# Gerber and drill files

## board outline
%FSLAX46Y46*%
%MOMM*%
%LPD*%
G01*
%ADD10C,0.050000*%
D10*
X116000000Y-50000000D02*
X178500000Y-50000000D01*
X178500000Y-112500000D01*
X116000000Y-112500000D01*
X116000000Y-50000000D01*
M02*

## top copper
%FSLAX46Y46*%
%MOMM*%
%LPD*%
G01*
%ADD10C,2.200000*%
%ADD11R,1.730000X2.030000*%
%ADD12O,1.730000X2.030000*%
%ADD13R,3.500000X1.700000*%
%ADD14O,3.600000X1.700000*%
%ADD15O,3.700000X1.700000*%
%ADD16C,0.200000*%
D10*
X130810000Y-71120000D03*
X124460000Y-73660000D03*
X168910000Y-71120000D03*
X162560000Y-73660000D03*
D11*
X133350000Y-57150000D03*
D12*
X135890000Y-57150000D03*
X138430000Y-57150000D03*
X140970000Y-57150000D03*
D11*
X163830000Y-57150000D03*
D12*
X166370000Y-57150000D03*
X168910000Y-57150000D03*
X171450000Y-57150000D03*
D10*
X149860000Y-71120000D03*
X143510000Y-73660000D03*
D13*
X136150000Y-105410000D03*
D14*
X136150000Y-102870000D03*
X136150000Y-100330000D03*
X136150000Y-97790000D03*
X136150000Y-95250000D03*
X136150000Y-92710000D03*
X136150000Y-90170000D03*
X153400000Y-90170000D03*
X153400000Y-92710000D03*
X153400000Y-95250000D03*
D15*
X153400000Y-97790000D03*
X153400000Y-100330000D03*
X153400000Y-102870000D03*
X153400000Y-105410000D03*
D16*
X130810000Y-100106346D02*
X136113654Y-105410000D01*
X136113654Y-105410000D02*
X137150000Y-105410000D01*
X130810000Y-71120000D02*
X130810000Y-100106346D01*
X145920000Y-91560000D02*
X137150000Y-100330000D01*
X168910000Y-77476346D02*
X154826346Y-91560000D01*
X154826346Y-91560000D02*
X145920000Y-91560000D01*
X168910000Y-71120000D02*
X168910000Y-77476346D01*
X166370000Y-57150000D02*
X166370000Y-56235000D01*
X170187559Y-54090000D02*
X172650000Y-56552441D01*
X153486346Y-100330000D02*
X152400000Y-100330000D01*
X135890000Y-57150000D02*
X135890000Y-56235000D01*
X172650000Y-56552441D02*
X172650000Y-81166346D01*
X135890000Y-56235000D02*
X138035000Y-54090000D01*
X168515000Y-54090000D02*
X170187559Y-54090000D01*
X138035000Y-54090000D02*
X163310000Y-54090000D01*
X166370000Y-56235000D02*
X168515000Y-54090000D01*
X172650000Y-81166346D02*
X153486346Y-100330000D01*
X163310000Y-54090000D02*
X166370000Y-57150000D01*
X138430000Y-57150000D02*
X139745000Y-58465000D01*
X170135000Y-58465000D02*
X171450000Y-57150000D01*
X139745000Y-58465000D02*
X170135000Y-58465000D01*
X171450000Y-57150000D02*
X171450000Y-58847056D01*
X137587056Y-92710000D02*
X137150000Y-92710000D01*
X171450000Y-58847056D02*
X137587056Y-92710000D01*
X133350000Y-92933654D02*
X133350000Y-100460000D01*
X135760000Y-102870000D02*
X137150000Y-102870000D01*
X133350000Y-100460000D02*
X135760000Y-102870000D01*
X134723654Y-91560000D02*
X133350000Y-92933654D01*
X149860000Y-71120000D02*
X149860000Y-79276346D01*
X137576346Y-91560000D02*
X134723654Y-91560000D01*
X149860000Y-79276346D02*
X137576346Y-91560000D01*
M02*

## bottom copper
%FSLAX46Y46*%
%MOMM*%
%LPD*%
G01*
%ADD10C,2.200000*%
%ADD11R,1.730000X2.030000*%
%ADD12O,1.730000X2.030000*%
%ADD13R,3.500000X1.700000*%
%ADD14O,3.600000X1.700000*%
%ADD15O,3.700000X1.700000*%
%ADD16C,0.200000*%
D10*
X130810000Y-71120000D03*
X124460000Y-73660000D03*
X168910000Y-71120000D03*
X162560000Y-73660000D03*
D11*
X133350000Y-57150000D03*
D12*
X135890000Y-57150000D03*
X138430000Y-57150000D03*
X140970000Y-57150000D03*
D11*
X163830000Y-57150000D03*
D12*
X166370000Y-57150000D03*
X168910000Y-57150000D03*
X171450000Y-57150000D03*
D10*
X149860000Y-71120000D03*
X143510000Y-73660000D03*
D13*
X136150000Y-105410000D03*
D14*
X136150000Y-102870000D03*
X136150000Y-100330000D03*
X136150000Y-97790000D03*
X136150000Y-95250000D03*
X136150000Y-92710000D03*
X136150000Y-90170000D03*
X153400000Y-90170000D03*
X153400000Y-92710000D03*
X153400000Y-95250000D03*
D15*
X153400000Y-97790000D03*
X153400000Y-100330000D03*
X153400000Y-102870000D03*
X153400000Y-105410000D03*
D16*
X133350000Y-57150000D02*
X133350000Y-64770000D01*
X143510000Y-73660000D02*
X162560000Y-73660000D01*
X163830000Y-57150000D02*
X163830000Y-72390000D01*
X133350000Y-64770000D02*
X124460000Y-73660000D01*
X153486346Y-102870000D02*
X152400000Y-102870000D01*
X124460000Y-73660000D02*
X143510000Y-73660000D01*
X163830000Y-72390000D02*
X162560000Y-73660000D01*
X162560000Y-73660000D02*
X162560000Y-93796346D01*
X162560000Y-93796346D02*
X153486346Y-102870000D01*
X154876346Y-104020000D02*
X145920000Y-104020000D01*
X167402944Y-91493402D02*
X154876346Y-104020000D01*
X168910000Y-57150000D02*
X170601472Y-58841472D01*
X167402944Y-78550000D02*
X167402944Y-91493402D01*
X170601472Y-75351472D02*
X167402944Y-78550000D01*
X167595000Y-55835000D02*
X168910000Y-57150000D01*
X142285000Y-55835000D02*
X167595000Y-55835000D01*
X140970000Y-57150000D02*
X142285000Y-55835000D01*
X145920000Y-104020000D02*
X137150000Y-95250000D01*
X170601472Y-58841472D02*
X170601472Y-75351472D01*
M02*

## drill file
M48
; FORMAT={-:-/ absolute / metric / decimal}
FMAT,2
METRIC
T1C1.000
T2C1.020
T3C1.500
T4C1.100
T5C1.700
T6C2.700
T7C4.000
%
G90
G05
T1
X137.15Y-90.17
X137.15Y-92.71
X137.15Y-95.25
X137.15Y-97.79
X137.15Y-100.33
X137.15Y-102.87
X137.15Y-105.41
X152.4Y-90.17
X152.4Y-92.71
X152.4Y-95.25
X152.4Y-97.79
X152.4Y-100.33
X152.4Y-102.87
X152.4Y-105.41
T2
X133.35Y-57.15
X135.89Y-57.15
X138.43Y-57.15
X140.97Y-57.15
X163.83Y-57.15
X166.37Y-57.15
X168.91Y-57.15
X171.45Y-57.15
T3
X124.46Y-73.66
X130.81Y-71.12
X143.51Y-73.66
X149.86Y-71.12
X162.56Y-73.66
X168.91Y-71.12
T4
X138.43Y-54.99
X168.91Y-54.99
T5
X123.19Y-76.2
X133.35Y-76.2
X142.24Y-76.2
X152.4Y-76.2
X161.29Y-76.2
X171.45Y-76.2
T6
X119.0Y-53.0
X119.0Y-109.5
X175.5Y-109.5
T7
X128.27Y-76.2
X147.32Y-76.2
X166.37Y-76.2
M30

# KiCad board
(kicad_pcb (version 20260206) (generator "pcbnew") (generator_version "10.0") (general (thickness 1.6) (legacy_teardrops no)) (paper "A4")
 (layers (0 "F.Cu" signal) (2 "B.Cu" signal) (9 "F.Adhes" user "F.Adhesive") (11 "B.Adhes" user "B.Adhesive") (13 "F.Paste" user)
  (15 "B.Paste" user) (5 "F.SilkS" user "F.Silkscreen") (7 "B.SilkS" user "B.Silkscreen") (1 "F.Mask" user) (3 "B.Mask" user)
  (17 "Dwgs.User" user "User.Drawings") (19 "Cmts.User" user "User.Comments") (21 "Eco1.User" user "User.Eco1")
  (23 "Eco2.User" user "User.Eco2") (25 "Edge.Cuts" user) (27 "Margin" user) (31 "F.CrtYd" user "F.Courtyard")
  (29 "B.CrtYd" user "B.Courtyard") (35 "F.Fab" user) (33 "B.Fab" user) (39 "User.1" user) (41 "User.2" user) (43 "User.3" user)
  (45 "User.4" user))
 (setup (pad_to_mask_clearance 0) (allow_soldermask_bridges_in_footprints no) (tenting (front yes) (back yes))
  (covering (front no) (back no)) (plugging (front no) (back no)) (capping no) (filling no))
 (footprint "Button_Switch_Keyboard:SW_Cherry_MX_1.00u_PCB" (layer "F.Cu") (at 130.81 71.12)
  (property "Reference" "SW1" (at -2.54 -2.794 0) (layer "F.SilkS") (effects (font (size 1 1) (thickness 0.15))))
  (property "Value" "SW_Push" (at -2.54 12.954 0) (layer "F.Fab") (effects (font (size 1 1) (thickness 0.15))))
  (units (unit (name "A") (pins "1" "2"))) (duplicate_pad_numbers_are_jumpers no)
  (pad "" np_thru_hole circle (at -7.62 5.08) (size 1.7 1.7) (drill 1.7) (layers "*.Cu" "*.Mask"))
  (pad "" np_thru_hole circle (at -2.54 5.08) (size 4 4) (drill 4) (layers "*.Cu" "*.Mask"))
  (pad "" np_thru_hole circle (at 2.54 5.08) (size 1.7 1.7) (drill 1.7) (layers "*.Cu" "*.Mask"))
  (pad "1" thru_hole circle (at 0 0) (size 2.2 2.2) (drill 1.5) (layers "*.Cu" "*.Mask") (remove_unused_layers no) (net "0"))
  (pad "2" thru_hole circle (at -6.35 2.54) (size 2.2 2.2) (drill 1.5) (layers "*.Cu" "*.Mask") (remove_unused_layers no) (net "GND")))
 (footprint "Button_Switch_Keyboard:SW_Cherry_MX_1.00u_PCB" (layer "F.Cu") (at 168.91 71.12)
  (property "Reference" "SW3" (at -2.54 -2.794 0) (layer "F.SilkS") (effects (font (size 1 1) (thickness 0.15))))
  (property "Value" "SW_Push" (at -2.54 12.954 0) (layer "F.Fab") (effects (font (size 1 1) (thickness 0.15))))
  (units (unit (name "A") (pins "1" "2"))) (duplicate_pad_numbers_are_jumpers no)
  (pad "" np_thru_hole circle (at -7.62 5.08) (size 1.7 1.7) (drill 1.7) (layers "*.Cu" "*.Mask"))
  (pad "" np_thru_hole circle (at -2.54 5.08) (size 4 4) (drill 4) (layers "*.Cu" "*.Mask"))
  (pad "" np_thru_hole circle (at 2.54 5.08) (size 1.7 1.7) (drill 1.7) (layers "*.Cu" "*.Mask"))
  (pad "1" thru_hole circle (at 0 0) (size 2.2 2.2) (drill 1.5) (layers "*.Cu" "*.Mask") (remove_unused_layers no) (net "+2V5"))
  (pad "2" thru_hole circle (at -6.35 2.54) (size 2.2 2.2) (drill 1.5) (layers "*.Cu" "*.Mask") (remove_unused_layers no) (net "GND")))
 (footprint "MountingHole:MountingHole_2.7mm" (layer "F.Cu") (at 119 109.5)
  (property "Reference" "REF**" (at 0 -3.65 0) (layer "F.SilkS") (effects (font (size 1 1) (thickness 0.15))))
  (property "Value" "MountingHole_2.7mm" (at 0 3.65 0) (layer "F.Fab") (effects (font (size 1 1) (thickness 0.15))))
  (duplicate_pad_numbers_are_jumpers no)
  (pad "" np_thru_hole circle (at 0 0) (size 2.7 2.7) (drill 2.7) (layers "*.Cu" "*.Mask")))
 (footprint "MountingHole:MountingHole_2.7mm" (layer "F.Cu") (at 175.5 109.5)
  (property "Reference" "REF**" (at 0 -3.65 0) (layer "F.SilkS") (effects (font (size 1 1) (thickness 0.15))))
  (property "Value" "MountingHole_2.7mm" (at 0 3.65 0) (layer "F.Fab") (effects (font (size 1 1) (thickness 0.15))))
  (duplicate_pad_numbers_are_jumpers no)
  (pad "" np_thru_hole circle (at 0 0) (size 2.7 2.7) (drill 2.7) (layers "*.Cu" "*.Mask")))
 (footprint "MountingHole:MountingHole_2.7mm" (layer "F.Cu") (at 119 53)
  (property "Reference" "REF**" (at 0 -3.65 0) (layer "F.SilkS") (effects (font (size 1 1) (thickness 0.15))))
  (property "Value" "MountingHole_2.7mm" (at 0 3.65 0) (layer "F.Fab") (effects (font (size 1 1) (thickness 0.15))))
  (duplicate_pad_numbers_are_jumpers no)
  (pad "" np_thru_hole circle (at 0 0) (size 2.7 2.7) (drill 2.7) (layers "*.Cu" "*.Mask")))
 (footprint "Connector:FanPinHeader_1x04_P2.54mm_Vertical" (layer "F.Cu") (at 133.35 57.15)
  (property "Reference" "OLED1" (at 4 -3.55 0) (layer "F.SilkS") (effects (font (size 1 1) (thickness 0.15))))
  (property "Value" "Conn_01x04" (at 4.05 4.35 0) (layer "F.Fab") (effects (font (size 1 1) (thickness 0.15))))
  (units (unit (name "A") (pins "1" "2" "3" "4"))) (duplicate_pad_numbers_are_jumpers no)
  (pad "" np_thru_hole circle (at 5.08 -2.16 90) (size 1.1 1.1) (drill 1.1) (layers "*.Cu" "*.Mask"))
  (pad "1" thru_hole rect (at 0 0 90) (size 2.03 1.73) (drill 1.02) (layers "*.Cu" "*.Mask") (remove_unused_layers no) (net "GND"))
  (pad "2" thru_hole oval (at 2.54 0 90) (size 2.03 1.73) (drill 1.02) (layers "*.Cu" "*.Mask") (remove_unused_layers no) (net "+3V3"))
  (pad "3" thru_hole oval (at 5.08 0 90) (size 2.03 1.73) (drill 1.02) (layers "*.Cu" "*.Mask") (remove_unused_layers no) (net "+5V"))
  (pad "4" thru_hole oval (at 7.62 0 90) (size 2.03 1.73) (drill 1.02) (layers "*.Cu" "*.Mask") (remove_unused_layers no) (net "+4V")))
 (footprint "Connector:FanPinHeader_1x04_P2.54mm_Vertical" (layer "F.Cu") (at 163.83 57.15)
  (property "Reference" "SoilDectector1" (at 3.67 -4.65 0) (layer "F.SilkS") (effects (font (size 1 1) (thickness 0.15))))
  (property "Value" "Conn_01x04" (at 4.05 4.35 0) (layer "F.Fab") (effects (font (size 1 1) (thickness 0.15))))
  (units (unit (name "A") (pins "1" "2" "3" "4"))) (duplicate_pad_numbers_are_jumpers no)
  (pad "" np_thru_hole circle (at 5.08 -2.16 90) (size 1.1 1.1) (drill 1.1) (layers "*.Cu" "*.Mask"))
  (pad "1" thru_hole rect (at 0 0 90) (size 2.03 1.73) (drill 1.02) (layers "*.Cu" "*.Mask") (remove_unused_layers no) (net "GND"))
  (pad "2" thru_hole oval (at 2.54 0 90) (size 2.03 1.73) (drill 1.02) (layers "*.Cu" "*.Mask") (remove_unused_layers no) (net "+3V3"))
  (pad "3" thru_hole oval (at 5.08 0 90) (size 2.03 1.73) (drill 1.02) (layers "*.Cu" "*.Mask") (remove_unused_layers no) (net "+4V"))
  (pad "4" thru_hole oval (at 7.62 0 90) (size 2.03 1.73) (drill 1.02) (layers "*.Cu" "*.Mask") (remove_unused_layers no) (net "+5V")))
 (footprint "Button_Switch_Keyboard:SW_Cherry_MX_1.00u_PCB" (layer "F.Cu") (at 149.86 71.12)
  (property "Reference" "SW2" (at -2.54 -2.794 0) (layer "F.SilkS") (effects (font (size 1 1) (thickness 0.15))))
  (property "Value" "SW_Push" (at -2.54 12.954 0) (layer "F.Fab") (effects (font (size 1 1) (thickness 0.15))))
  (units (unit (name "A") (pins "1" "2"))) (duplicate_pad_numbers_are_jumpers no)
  (pad "" np_thru_hole circle (at -7.62 5.08) (size 1.7 1.7) (drill 1.7) (layers "*.Cu" "*.Mask"))
  (pad "" np_thru_hole circle (at -2.54 5.08) (size 4 4) (drill 4) (layers "*.Cu" "*.Mask"))
  (pad "" np_thru_hole circle (at 2.54 5.08) (size 1.7 1.7) (drill 1.7) (layers "*.Cu" "*.Mask"))
  (pad "1" thru_hole circle (at 0 0) (size 2.2 2.2) (drill 1.5) (layers "*.Cu" "*.Mask") (remove_unused_layers no) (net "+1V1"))
  (pad "2" thru_hole circle (at -6.35 2.54) (size 2.2 2.2) (drill 1.5) (layers "*.Cu" "*.Mask") (remove_unused_layers no) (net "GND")))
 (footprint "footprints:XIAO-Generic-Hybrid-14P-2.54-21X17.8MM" (layer "B.Cu") (at 144.775 97.79)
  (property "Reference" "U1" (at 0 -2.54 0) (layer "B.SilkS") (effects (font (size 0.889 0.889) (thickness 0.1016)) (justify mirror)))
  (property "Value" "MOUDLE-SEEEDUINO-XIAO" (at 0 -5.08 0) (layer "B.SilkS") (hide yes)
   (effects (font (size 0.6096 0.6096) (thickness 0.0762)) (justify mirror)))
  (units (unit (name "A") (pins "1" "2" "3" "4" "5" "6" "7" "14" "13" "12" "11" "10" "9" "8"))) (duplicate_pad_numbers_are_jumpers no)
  (pad "1" thru_hole rect (at -7.625 7.62) (size 3.5 1.7) (drill 1 (offset -1 0)) (layers "*.Cu" "*.Mask") (remove_unused_layers no)
   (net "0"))
  (pad "2" thru_hole oval (at -7.625 5.08) (size 3.6 1.7) (drill 1 (offset -1 0)) (layers "*.Cu" "*.Mask") (remove_unused_layers no)
   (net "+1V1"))
  (pad "3" thru_hole oval (at -7.625 2.54) (size 3.6 1.7) (drill 1 (offset -1 0)) (layers "*.Cu" "*.Mask") (remove_unused_layers no)
   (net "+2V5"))
  (pad "4" thru_hole oval (at -7.625 0) (size 3.6 1.7) (drill 1 (offset -1 0)) (layers "*.Cu" "*.Mask") (remove_unused_layers no)
   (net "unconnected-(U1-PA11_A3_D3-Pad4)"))
  (pad "5" thru_hole oval (at -7.625 -2.54) (size 3.6 1.7) (drill 1 (offset -1 0)) (layers "*.Cu" "*.Mask") (remove_unused_layers no)
   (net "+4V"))
  (pad "6" thru_hole oval (at -7.625 -5.08 180) (size 3.6 1.7) (drill 1 (offset 1 0)) (layers "*.Cu" "*.Mask") (remove_unused_layers no)
   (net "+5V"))
  (pad "7" thru_hole oval (at -7.625 -7.62) (size 3.6 1.7) (drill 1 (offset -1 0)) (layers "*.Cu" "*.Mask") (remove_unused_layers no)
   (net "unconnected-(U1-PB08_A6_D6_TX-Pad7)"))
  (pad "8" thru_hole oval (at 7.625 -7.62) (size 3.6 1.7) (drill 1 (offset 1 0)) (layers "*.Cu" "*.Mask") (remove_unused_layers no)
   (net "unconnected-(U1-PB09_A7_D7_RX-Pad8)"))
  (pad "9" thru_hole oval (at 7.625 -5.08) (size 3.6 1.7) (drill 1 (offset 1 0)) (layers "*.Cu" "*.Mask") (remove_unused_layers no)
   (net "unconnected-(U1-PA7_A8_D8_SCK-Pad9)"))
  (pad "10" thru_hole oval (at 7.625 -2.54) (size 3.6 1.7) (drill 1 (offset 1 0)) (layers "*.Cu" "*.Mask") (remove_unused_layers no)
   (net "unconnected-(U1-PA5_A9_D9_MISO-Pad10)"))
  (pad "11" thru_hole oval (at 7.625 0) (size 3.7 1.7) (drill 1 (offset 1 0)) (layers "*.Cu" "*.Mask") (remove_unused_layers no)
   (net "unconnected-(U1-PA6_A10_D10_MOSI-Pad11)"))
  (pad "12" thru_hole oval (at 7.625 2.54) (size 3.7 1.7) (drill 1 (offset 1 0)) (layers "*.Cu" "*.Mask") (remove_unused_layers no)
   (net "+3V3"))
  (pad "13" thru_hole oval (at 7.625 5.08) (size 3.7 1.7) (drill 1 (offset 1 0)) (layers "*.Cu" "*.Mask") (remove_unused_layers no)
   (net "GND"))
  (pad "14" thru_hole oval (at 7.625 7.62) (size 3.7 1.7) (drill 1 (offset 1 0)) (layers "*.Cu" "*.Mask") (remove_unused_layers no)
   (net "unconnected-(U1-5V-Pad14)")))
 (gr_rect (start 116 50) (end 178.5 112.5) (stroke (width 0.05) (type default)) (fill no) (layer "Edge.Cuts"))
 (segment (start 130.81 100.106346) (end 136.113654 105.41) (width 0.2) (layer "F.Cu") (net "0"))
 (segment (start 136.113654 105.41) (end 137.15 105.41) (width 0.2) (layer "F.Cu") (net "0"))
 (segment (start 130.81 71.12) (end 130.81 100.106346) (width 0.2) (layer "F.Cu") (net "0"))
 (segment (start 133.35 57.15) (end 133.35 64.77) (width 0.2) (layer "B.Cu") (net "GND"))
 (segment (start 143.51 73.66) (end 162.56 73.66) (width 0.2) (layer "B.Cu") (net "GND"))
 (segment (start 163.83 57.15) (end 163.83 72.39) (width 0.2) (layer "B.Cu") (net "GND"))
 (segment (start 133.35 64.77) (end 124.46 73.66) (width 0.2) (layer "B.Cu") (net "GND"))
 (segment (start 153.486346 102.87) (end 152.4 102.87) (width 0.2) (layer "B.Cu") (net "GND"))
 (segment (start 124.46 73.66) (end 143.51 73.66) (width 0.2) (layer "B.Cu") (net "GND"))
 (segment (start 163.83 72.39) (end 162.56 73.66) (width 0.2) (layer "B.Cu") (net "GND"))
 (segment (start 162.56 73.66) (end 162.56 93.796346) (width 0.2) (layer "B.Cu") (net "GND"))
 (segment (start 162.56 93.796346) (end 153.486346 102.87) (width 0.2) (layer "B.Cu") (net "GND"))
 (segment (start 145.92 91.56) (end 137.15 100.33) (width 0.2) (layer "F.Cu") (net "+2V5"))
 (segment (start 168.91 77.476346) (end 154.826346 91.56) (width 0.2) (layer "F.Cu") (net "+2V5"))
 (segment (start 154.826346 91.56) (end 145.92 91.56) (width 0.2) (layer "F.Cu") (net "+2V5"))
 (segment (start 168.91 71.12) (end 168.91 77.476346) (width 0.2) (layer "F.Cu") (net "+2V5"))
 (segment (start 166.37 57.15) (end 166.37 56.235) (width 0.2) (layer "F.Cu") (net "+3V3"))
 (segment (start 170.187559 54.09) (end 172.65 56.552441) (width 0.2) (layer "F.Cu") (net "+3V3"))
 (segment (start 153.486346 100.33) (end 152.4 100.33) (width 0.2) (layer "F.Cu") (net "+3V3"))
 (segment (start 135.89 57.15) (end 135.89 56.235) (width 0.2) (layer "F.Cu") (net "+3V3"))
 (segment (start 172.65 56.552441) (end 172.65 81.166346) (width 0.2) (layer "F.Cu") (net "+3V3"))
 (segment (start 135.89 56.235) (end 138.035 54.09) (width 0.2) (layer "F.Cu") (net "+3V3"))
 (segment (start 168.515 54.09) (end 170.187559 54.09) (width 0.2) (layer "F.Cu") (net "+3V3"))
 (segment (start 138.035 54.09) (end 163.31 54.09) (width 0.2) (layer "F.Cu") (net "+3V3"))
 (segment (start 166.37 56.235) (end 168.515 54.09) (width 0.2) (layer "F.Cu") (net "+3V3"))
 (segment (start 172.65 81.166346) (end 153.486346 100.33) (width 0.2) (layer "F.Cu") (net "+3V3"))
 (segment (start 163.31 54.09) (end 166.37 57.15) (width 0.2) (layer "F.Cu") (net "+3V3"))
 (segment (start 138.43 57.15) (end 139.745 58.465) (width 0.2) (layer "F.Cu") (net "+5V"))
 (segment (start 170.135 58.465) (end 171.45 57.15) (width 0.2) (layer "F.Cu") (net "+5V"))
 (segment (start 139.745 58.465) (end 170.135 58.465) (width 0.2) (layer "F.Cu") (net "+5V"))
 (segment (start 171.45 57.15) (end 171.45 58.847056) (width 0.2) (layer "F.Cu") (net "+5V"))
 (segment (start 137.587056 92.71) (end 137.15 92.71) (width 0.2) (layer "F.Cu") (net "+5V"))
 (segment (start 171.45 58.847056) (end 137.587056 92.71) (width 0.2) (layer "F.Cu") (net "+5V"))
 (segment (start 154.876346 104.02) (end 145.92 104.02) (width 0.2) (layer "B.Cu") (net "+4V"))
 (segment (start 167.402944 91.493402) (end 154.876346 104.02) (width 0.2) (layer "B.Cu") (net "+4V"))
 (segment (start 168.91 57.15) (end 170.601472 58.841472) (width 0.2) (layer "B.Cu") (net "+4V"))
 (segment (start 167.402944 78.55) (end 167.402944 91.493402) (width 0.2) (layer "B.Cu") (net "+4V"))
 (segment (start 170.601472 75.351472) (end 167.402944 78.55) (width 0.2) (layer "B.Cu") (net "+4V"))
 (segment (start 167.595 55.835) (end 168.91 57.15) (width 0.2) (layer "B.Cu") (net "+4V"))
 (segment (start 142.285 55.835) (end 167.595 55.835) (width 0.2) (layer "B.Cu") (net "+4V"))
 (segment (start 140.97 57.15) (end 142.285 55.835) (width 0.2) (layer "B.Cu") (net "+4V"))
 (segment (start 145.92 104.02) (end 137.15 95.25) (width 0.2) (layer "B.Cu") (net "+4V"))
 (segment (start 170.601472 58.841472) (end 170.601472 75.351472) (width 0.2) (layer "B.Cu") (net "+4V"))
 (segment (start 133.35 92.933654) (end 133.35 100.46) (width 0.2) (layer "F.Cu") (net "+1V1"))
 (segment (start 135.76 102.87) (end 137.15 102.87) (width 0.2) (layer "F.Cu") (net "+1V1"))
 (segment (start 133.35 100.46) (end 135.76 102.87) (width 0.2) (layer "F.Cu") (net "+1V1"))
 (segment (start 134.723654 91.56) (end 133.35 92.933654) (width 0.2) (layer "F.Cu") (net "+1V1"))
 (segment (start 149.86 71.12) (end 149.86 79.276346) (width 0.2) (layer "F.Cu") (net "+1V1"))
 (segment (start 137.576346 91.56) (end 134.723654 91.56) (width 0.2) (layer "F.Cu") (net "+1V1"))
 (segment (start 149.86 79.276346) (end 137.576346 91.56) (width 0.2) (layer "F.Cu") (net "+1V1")))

